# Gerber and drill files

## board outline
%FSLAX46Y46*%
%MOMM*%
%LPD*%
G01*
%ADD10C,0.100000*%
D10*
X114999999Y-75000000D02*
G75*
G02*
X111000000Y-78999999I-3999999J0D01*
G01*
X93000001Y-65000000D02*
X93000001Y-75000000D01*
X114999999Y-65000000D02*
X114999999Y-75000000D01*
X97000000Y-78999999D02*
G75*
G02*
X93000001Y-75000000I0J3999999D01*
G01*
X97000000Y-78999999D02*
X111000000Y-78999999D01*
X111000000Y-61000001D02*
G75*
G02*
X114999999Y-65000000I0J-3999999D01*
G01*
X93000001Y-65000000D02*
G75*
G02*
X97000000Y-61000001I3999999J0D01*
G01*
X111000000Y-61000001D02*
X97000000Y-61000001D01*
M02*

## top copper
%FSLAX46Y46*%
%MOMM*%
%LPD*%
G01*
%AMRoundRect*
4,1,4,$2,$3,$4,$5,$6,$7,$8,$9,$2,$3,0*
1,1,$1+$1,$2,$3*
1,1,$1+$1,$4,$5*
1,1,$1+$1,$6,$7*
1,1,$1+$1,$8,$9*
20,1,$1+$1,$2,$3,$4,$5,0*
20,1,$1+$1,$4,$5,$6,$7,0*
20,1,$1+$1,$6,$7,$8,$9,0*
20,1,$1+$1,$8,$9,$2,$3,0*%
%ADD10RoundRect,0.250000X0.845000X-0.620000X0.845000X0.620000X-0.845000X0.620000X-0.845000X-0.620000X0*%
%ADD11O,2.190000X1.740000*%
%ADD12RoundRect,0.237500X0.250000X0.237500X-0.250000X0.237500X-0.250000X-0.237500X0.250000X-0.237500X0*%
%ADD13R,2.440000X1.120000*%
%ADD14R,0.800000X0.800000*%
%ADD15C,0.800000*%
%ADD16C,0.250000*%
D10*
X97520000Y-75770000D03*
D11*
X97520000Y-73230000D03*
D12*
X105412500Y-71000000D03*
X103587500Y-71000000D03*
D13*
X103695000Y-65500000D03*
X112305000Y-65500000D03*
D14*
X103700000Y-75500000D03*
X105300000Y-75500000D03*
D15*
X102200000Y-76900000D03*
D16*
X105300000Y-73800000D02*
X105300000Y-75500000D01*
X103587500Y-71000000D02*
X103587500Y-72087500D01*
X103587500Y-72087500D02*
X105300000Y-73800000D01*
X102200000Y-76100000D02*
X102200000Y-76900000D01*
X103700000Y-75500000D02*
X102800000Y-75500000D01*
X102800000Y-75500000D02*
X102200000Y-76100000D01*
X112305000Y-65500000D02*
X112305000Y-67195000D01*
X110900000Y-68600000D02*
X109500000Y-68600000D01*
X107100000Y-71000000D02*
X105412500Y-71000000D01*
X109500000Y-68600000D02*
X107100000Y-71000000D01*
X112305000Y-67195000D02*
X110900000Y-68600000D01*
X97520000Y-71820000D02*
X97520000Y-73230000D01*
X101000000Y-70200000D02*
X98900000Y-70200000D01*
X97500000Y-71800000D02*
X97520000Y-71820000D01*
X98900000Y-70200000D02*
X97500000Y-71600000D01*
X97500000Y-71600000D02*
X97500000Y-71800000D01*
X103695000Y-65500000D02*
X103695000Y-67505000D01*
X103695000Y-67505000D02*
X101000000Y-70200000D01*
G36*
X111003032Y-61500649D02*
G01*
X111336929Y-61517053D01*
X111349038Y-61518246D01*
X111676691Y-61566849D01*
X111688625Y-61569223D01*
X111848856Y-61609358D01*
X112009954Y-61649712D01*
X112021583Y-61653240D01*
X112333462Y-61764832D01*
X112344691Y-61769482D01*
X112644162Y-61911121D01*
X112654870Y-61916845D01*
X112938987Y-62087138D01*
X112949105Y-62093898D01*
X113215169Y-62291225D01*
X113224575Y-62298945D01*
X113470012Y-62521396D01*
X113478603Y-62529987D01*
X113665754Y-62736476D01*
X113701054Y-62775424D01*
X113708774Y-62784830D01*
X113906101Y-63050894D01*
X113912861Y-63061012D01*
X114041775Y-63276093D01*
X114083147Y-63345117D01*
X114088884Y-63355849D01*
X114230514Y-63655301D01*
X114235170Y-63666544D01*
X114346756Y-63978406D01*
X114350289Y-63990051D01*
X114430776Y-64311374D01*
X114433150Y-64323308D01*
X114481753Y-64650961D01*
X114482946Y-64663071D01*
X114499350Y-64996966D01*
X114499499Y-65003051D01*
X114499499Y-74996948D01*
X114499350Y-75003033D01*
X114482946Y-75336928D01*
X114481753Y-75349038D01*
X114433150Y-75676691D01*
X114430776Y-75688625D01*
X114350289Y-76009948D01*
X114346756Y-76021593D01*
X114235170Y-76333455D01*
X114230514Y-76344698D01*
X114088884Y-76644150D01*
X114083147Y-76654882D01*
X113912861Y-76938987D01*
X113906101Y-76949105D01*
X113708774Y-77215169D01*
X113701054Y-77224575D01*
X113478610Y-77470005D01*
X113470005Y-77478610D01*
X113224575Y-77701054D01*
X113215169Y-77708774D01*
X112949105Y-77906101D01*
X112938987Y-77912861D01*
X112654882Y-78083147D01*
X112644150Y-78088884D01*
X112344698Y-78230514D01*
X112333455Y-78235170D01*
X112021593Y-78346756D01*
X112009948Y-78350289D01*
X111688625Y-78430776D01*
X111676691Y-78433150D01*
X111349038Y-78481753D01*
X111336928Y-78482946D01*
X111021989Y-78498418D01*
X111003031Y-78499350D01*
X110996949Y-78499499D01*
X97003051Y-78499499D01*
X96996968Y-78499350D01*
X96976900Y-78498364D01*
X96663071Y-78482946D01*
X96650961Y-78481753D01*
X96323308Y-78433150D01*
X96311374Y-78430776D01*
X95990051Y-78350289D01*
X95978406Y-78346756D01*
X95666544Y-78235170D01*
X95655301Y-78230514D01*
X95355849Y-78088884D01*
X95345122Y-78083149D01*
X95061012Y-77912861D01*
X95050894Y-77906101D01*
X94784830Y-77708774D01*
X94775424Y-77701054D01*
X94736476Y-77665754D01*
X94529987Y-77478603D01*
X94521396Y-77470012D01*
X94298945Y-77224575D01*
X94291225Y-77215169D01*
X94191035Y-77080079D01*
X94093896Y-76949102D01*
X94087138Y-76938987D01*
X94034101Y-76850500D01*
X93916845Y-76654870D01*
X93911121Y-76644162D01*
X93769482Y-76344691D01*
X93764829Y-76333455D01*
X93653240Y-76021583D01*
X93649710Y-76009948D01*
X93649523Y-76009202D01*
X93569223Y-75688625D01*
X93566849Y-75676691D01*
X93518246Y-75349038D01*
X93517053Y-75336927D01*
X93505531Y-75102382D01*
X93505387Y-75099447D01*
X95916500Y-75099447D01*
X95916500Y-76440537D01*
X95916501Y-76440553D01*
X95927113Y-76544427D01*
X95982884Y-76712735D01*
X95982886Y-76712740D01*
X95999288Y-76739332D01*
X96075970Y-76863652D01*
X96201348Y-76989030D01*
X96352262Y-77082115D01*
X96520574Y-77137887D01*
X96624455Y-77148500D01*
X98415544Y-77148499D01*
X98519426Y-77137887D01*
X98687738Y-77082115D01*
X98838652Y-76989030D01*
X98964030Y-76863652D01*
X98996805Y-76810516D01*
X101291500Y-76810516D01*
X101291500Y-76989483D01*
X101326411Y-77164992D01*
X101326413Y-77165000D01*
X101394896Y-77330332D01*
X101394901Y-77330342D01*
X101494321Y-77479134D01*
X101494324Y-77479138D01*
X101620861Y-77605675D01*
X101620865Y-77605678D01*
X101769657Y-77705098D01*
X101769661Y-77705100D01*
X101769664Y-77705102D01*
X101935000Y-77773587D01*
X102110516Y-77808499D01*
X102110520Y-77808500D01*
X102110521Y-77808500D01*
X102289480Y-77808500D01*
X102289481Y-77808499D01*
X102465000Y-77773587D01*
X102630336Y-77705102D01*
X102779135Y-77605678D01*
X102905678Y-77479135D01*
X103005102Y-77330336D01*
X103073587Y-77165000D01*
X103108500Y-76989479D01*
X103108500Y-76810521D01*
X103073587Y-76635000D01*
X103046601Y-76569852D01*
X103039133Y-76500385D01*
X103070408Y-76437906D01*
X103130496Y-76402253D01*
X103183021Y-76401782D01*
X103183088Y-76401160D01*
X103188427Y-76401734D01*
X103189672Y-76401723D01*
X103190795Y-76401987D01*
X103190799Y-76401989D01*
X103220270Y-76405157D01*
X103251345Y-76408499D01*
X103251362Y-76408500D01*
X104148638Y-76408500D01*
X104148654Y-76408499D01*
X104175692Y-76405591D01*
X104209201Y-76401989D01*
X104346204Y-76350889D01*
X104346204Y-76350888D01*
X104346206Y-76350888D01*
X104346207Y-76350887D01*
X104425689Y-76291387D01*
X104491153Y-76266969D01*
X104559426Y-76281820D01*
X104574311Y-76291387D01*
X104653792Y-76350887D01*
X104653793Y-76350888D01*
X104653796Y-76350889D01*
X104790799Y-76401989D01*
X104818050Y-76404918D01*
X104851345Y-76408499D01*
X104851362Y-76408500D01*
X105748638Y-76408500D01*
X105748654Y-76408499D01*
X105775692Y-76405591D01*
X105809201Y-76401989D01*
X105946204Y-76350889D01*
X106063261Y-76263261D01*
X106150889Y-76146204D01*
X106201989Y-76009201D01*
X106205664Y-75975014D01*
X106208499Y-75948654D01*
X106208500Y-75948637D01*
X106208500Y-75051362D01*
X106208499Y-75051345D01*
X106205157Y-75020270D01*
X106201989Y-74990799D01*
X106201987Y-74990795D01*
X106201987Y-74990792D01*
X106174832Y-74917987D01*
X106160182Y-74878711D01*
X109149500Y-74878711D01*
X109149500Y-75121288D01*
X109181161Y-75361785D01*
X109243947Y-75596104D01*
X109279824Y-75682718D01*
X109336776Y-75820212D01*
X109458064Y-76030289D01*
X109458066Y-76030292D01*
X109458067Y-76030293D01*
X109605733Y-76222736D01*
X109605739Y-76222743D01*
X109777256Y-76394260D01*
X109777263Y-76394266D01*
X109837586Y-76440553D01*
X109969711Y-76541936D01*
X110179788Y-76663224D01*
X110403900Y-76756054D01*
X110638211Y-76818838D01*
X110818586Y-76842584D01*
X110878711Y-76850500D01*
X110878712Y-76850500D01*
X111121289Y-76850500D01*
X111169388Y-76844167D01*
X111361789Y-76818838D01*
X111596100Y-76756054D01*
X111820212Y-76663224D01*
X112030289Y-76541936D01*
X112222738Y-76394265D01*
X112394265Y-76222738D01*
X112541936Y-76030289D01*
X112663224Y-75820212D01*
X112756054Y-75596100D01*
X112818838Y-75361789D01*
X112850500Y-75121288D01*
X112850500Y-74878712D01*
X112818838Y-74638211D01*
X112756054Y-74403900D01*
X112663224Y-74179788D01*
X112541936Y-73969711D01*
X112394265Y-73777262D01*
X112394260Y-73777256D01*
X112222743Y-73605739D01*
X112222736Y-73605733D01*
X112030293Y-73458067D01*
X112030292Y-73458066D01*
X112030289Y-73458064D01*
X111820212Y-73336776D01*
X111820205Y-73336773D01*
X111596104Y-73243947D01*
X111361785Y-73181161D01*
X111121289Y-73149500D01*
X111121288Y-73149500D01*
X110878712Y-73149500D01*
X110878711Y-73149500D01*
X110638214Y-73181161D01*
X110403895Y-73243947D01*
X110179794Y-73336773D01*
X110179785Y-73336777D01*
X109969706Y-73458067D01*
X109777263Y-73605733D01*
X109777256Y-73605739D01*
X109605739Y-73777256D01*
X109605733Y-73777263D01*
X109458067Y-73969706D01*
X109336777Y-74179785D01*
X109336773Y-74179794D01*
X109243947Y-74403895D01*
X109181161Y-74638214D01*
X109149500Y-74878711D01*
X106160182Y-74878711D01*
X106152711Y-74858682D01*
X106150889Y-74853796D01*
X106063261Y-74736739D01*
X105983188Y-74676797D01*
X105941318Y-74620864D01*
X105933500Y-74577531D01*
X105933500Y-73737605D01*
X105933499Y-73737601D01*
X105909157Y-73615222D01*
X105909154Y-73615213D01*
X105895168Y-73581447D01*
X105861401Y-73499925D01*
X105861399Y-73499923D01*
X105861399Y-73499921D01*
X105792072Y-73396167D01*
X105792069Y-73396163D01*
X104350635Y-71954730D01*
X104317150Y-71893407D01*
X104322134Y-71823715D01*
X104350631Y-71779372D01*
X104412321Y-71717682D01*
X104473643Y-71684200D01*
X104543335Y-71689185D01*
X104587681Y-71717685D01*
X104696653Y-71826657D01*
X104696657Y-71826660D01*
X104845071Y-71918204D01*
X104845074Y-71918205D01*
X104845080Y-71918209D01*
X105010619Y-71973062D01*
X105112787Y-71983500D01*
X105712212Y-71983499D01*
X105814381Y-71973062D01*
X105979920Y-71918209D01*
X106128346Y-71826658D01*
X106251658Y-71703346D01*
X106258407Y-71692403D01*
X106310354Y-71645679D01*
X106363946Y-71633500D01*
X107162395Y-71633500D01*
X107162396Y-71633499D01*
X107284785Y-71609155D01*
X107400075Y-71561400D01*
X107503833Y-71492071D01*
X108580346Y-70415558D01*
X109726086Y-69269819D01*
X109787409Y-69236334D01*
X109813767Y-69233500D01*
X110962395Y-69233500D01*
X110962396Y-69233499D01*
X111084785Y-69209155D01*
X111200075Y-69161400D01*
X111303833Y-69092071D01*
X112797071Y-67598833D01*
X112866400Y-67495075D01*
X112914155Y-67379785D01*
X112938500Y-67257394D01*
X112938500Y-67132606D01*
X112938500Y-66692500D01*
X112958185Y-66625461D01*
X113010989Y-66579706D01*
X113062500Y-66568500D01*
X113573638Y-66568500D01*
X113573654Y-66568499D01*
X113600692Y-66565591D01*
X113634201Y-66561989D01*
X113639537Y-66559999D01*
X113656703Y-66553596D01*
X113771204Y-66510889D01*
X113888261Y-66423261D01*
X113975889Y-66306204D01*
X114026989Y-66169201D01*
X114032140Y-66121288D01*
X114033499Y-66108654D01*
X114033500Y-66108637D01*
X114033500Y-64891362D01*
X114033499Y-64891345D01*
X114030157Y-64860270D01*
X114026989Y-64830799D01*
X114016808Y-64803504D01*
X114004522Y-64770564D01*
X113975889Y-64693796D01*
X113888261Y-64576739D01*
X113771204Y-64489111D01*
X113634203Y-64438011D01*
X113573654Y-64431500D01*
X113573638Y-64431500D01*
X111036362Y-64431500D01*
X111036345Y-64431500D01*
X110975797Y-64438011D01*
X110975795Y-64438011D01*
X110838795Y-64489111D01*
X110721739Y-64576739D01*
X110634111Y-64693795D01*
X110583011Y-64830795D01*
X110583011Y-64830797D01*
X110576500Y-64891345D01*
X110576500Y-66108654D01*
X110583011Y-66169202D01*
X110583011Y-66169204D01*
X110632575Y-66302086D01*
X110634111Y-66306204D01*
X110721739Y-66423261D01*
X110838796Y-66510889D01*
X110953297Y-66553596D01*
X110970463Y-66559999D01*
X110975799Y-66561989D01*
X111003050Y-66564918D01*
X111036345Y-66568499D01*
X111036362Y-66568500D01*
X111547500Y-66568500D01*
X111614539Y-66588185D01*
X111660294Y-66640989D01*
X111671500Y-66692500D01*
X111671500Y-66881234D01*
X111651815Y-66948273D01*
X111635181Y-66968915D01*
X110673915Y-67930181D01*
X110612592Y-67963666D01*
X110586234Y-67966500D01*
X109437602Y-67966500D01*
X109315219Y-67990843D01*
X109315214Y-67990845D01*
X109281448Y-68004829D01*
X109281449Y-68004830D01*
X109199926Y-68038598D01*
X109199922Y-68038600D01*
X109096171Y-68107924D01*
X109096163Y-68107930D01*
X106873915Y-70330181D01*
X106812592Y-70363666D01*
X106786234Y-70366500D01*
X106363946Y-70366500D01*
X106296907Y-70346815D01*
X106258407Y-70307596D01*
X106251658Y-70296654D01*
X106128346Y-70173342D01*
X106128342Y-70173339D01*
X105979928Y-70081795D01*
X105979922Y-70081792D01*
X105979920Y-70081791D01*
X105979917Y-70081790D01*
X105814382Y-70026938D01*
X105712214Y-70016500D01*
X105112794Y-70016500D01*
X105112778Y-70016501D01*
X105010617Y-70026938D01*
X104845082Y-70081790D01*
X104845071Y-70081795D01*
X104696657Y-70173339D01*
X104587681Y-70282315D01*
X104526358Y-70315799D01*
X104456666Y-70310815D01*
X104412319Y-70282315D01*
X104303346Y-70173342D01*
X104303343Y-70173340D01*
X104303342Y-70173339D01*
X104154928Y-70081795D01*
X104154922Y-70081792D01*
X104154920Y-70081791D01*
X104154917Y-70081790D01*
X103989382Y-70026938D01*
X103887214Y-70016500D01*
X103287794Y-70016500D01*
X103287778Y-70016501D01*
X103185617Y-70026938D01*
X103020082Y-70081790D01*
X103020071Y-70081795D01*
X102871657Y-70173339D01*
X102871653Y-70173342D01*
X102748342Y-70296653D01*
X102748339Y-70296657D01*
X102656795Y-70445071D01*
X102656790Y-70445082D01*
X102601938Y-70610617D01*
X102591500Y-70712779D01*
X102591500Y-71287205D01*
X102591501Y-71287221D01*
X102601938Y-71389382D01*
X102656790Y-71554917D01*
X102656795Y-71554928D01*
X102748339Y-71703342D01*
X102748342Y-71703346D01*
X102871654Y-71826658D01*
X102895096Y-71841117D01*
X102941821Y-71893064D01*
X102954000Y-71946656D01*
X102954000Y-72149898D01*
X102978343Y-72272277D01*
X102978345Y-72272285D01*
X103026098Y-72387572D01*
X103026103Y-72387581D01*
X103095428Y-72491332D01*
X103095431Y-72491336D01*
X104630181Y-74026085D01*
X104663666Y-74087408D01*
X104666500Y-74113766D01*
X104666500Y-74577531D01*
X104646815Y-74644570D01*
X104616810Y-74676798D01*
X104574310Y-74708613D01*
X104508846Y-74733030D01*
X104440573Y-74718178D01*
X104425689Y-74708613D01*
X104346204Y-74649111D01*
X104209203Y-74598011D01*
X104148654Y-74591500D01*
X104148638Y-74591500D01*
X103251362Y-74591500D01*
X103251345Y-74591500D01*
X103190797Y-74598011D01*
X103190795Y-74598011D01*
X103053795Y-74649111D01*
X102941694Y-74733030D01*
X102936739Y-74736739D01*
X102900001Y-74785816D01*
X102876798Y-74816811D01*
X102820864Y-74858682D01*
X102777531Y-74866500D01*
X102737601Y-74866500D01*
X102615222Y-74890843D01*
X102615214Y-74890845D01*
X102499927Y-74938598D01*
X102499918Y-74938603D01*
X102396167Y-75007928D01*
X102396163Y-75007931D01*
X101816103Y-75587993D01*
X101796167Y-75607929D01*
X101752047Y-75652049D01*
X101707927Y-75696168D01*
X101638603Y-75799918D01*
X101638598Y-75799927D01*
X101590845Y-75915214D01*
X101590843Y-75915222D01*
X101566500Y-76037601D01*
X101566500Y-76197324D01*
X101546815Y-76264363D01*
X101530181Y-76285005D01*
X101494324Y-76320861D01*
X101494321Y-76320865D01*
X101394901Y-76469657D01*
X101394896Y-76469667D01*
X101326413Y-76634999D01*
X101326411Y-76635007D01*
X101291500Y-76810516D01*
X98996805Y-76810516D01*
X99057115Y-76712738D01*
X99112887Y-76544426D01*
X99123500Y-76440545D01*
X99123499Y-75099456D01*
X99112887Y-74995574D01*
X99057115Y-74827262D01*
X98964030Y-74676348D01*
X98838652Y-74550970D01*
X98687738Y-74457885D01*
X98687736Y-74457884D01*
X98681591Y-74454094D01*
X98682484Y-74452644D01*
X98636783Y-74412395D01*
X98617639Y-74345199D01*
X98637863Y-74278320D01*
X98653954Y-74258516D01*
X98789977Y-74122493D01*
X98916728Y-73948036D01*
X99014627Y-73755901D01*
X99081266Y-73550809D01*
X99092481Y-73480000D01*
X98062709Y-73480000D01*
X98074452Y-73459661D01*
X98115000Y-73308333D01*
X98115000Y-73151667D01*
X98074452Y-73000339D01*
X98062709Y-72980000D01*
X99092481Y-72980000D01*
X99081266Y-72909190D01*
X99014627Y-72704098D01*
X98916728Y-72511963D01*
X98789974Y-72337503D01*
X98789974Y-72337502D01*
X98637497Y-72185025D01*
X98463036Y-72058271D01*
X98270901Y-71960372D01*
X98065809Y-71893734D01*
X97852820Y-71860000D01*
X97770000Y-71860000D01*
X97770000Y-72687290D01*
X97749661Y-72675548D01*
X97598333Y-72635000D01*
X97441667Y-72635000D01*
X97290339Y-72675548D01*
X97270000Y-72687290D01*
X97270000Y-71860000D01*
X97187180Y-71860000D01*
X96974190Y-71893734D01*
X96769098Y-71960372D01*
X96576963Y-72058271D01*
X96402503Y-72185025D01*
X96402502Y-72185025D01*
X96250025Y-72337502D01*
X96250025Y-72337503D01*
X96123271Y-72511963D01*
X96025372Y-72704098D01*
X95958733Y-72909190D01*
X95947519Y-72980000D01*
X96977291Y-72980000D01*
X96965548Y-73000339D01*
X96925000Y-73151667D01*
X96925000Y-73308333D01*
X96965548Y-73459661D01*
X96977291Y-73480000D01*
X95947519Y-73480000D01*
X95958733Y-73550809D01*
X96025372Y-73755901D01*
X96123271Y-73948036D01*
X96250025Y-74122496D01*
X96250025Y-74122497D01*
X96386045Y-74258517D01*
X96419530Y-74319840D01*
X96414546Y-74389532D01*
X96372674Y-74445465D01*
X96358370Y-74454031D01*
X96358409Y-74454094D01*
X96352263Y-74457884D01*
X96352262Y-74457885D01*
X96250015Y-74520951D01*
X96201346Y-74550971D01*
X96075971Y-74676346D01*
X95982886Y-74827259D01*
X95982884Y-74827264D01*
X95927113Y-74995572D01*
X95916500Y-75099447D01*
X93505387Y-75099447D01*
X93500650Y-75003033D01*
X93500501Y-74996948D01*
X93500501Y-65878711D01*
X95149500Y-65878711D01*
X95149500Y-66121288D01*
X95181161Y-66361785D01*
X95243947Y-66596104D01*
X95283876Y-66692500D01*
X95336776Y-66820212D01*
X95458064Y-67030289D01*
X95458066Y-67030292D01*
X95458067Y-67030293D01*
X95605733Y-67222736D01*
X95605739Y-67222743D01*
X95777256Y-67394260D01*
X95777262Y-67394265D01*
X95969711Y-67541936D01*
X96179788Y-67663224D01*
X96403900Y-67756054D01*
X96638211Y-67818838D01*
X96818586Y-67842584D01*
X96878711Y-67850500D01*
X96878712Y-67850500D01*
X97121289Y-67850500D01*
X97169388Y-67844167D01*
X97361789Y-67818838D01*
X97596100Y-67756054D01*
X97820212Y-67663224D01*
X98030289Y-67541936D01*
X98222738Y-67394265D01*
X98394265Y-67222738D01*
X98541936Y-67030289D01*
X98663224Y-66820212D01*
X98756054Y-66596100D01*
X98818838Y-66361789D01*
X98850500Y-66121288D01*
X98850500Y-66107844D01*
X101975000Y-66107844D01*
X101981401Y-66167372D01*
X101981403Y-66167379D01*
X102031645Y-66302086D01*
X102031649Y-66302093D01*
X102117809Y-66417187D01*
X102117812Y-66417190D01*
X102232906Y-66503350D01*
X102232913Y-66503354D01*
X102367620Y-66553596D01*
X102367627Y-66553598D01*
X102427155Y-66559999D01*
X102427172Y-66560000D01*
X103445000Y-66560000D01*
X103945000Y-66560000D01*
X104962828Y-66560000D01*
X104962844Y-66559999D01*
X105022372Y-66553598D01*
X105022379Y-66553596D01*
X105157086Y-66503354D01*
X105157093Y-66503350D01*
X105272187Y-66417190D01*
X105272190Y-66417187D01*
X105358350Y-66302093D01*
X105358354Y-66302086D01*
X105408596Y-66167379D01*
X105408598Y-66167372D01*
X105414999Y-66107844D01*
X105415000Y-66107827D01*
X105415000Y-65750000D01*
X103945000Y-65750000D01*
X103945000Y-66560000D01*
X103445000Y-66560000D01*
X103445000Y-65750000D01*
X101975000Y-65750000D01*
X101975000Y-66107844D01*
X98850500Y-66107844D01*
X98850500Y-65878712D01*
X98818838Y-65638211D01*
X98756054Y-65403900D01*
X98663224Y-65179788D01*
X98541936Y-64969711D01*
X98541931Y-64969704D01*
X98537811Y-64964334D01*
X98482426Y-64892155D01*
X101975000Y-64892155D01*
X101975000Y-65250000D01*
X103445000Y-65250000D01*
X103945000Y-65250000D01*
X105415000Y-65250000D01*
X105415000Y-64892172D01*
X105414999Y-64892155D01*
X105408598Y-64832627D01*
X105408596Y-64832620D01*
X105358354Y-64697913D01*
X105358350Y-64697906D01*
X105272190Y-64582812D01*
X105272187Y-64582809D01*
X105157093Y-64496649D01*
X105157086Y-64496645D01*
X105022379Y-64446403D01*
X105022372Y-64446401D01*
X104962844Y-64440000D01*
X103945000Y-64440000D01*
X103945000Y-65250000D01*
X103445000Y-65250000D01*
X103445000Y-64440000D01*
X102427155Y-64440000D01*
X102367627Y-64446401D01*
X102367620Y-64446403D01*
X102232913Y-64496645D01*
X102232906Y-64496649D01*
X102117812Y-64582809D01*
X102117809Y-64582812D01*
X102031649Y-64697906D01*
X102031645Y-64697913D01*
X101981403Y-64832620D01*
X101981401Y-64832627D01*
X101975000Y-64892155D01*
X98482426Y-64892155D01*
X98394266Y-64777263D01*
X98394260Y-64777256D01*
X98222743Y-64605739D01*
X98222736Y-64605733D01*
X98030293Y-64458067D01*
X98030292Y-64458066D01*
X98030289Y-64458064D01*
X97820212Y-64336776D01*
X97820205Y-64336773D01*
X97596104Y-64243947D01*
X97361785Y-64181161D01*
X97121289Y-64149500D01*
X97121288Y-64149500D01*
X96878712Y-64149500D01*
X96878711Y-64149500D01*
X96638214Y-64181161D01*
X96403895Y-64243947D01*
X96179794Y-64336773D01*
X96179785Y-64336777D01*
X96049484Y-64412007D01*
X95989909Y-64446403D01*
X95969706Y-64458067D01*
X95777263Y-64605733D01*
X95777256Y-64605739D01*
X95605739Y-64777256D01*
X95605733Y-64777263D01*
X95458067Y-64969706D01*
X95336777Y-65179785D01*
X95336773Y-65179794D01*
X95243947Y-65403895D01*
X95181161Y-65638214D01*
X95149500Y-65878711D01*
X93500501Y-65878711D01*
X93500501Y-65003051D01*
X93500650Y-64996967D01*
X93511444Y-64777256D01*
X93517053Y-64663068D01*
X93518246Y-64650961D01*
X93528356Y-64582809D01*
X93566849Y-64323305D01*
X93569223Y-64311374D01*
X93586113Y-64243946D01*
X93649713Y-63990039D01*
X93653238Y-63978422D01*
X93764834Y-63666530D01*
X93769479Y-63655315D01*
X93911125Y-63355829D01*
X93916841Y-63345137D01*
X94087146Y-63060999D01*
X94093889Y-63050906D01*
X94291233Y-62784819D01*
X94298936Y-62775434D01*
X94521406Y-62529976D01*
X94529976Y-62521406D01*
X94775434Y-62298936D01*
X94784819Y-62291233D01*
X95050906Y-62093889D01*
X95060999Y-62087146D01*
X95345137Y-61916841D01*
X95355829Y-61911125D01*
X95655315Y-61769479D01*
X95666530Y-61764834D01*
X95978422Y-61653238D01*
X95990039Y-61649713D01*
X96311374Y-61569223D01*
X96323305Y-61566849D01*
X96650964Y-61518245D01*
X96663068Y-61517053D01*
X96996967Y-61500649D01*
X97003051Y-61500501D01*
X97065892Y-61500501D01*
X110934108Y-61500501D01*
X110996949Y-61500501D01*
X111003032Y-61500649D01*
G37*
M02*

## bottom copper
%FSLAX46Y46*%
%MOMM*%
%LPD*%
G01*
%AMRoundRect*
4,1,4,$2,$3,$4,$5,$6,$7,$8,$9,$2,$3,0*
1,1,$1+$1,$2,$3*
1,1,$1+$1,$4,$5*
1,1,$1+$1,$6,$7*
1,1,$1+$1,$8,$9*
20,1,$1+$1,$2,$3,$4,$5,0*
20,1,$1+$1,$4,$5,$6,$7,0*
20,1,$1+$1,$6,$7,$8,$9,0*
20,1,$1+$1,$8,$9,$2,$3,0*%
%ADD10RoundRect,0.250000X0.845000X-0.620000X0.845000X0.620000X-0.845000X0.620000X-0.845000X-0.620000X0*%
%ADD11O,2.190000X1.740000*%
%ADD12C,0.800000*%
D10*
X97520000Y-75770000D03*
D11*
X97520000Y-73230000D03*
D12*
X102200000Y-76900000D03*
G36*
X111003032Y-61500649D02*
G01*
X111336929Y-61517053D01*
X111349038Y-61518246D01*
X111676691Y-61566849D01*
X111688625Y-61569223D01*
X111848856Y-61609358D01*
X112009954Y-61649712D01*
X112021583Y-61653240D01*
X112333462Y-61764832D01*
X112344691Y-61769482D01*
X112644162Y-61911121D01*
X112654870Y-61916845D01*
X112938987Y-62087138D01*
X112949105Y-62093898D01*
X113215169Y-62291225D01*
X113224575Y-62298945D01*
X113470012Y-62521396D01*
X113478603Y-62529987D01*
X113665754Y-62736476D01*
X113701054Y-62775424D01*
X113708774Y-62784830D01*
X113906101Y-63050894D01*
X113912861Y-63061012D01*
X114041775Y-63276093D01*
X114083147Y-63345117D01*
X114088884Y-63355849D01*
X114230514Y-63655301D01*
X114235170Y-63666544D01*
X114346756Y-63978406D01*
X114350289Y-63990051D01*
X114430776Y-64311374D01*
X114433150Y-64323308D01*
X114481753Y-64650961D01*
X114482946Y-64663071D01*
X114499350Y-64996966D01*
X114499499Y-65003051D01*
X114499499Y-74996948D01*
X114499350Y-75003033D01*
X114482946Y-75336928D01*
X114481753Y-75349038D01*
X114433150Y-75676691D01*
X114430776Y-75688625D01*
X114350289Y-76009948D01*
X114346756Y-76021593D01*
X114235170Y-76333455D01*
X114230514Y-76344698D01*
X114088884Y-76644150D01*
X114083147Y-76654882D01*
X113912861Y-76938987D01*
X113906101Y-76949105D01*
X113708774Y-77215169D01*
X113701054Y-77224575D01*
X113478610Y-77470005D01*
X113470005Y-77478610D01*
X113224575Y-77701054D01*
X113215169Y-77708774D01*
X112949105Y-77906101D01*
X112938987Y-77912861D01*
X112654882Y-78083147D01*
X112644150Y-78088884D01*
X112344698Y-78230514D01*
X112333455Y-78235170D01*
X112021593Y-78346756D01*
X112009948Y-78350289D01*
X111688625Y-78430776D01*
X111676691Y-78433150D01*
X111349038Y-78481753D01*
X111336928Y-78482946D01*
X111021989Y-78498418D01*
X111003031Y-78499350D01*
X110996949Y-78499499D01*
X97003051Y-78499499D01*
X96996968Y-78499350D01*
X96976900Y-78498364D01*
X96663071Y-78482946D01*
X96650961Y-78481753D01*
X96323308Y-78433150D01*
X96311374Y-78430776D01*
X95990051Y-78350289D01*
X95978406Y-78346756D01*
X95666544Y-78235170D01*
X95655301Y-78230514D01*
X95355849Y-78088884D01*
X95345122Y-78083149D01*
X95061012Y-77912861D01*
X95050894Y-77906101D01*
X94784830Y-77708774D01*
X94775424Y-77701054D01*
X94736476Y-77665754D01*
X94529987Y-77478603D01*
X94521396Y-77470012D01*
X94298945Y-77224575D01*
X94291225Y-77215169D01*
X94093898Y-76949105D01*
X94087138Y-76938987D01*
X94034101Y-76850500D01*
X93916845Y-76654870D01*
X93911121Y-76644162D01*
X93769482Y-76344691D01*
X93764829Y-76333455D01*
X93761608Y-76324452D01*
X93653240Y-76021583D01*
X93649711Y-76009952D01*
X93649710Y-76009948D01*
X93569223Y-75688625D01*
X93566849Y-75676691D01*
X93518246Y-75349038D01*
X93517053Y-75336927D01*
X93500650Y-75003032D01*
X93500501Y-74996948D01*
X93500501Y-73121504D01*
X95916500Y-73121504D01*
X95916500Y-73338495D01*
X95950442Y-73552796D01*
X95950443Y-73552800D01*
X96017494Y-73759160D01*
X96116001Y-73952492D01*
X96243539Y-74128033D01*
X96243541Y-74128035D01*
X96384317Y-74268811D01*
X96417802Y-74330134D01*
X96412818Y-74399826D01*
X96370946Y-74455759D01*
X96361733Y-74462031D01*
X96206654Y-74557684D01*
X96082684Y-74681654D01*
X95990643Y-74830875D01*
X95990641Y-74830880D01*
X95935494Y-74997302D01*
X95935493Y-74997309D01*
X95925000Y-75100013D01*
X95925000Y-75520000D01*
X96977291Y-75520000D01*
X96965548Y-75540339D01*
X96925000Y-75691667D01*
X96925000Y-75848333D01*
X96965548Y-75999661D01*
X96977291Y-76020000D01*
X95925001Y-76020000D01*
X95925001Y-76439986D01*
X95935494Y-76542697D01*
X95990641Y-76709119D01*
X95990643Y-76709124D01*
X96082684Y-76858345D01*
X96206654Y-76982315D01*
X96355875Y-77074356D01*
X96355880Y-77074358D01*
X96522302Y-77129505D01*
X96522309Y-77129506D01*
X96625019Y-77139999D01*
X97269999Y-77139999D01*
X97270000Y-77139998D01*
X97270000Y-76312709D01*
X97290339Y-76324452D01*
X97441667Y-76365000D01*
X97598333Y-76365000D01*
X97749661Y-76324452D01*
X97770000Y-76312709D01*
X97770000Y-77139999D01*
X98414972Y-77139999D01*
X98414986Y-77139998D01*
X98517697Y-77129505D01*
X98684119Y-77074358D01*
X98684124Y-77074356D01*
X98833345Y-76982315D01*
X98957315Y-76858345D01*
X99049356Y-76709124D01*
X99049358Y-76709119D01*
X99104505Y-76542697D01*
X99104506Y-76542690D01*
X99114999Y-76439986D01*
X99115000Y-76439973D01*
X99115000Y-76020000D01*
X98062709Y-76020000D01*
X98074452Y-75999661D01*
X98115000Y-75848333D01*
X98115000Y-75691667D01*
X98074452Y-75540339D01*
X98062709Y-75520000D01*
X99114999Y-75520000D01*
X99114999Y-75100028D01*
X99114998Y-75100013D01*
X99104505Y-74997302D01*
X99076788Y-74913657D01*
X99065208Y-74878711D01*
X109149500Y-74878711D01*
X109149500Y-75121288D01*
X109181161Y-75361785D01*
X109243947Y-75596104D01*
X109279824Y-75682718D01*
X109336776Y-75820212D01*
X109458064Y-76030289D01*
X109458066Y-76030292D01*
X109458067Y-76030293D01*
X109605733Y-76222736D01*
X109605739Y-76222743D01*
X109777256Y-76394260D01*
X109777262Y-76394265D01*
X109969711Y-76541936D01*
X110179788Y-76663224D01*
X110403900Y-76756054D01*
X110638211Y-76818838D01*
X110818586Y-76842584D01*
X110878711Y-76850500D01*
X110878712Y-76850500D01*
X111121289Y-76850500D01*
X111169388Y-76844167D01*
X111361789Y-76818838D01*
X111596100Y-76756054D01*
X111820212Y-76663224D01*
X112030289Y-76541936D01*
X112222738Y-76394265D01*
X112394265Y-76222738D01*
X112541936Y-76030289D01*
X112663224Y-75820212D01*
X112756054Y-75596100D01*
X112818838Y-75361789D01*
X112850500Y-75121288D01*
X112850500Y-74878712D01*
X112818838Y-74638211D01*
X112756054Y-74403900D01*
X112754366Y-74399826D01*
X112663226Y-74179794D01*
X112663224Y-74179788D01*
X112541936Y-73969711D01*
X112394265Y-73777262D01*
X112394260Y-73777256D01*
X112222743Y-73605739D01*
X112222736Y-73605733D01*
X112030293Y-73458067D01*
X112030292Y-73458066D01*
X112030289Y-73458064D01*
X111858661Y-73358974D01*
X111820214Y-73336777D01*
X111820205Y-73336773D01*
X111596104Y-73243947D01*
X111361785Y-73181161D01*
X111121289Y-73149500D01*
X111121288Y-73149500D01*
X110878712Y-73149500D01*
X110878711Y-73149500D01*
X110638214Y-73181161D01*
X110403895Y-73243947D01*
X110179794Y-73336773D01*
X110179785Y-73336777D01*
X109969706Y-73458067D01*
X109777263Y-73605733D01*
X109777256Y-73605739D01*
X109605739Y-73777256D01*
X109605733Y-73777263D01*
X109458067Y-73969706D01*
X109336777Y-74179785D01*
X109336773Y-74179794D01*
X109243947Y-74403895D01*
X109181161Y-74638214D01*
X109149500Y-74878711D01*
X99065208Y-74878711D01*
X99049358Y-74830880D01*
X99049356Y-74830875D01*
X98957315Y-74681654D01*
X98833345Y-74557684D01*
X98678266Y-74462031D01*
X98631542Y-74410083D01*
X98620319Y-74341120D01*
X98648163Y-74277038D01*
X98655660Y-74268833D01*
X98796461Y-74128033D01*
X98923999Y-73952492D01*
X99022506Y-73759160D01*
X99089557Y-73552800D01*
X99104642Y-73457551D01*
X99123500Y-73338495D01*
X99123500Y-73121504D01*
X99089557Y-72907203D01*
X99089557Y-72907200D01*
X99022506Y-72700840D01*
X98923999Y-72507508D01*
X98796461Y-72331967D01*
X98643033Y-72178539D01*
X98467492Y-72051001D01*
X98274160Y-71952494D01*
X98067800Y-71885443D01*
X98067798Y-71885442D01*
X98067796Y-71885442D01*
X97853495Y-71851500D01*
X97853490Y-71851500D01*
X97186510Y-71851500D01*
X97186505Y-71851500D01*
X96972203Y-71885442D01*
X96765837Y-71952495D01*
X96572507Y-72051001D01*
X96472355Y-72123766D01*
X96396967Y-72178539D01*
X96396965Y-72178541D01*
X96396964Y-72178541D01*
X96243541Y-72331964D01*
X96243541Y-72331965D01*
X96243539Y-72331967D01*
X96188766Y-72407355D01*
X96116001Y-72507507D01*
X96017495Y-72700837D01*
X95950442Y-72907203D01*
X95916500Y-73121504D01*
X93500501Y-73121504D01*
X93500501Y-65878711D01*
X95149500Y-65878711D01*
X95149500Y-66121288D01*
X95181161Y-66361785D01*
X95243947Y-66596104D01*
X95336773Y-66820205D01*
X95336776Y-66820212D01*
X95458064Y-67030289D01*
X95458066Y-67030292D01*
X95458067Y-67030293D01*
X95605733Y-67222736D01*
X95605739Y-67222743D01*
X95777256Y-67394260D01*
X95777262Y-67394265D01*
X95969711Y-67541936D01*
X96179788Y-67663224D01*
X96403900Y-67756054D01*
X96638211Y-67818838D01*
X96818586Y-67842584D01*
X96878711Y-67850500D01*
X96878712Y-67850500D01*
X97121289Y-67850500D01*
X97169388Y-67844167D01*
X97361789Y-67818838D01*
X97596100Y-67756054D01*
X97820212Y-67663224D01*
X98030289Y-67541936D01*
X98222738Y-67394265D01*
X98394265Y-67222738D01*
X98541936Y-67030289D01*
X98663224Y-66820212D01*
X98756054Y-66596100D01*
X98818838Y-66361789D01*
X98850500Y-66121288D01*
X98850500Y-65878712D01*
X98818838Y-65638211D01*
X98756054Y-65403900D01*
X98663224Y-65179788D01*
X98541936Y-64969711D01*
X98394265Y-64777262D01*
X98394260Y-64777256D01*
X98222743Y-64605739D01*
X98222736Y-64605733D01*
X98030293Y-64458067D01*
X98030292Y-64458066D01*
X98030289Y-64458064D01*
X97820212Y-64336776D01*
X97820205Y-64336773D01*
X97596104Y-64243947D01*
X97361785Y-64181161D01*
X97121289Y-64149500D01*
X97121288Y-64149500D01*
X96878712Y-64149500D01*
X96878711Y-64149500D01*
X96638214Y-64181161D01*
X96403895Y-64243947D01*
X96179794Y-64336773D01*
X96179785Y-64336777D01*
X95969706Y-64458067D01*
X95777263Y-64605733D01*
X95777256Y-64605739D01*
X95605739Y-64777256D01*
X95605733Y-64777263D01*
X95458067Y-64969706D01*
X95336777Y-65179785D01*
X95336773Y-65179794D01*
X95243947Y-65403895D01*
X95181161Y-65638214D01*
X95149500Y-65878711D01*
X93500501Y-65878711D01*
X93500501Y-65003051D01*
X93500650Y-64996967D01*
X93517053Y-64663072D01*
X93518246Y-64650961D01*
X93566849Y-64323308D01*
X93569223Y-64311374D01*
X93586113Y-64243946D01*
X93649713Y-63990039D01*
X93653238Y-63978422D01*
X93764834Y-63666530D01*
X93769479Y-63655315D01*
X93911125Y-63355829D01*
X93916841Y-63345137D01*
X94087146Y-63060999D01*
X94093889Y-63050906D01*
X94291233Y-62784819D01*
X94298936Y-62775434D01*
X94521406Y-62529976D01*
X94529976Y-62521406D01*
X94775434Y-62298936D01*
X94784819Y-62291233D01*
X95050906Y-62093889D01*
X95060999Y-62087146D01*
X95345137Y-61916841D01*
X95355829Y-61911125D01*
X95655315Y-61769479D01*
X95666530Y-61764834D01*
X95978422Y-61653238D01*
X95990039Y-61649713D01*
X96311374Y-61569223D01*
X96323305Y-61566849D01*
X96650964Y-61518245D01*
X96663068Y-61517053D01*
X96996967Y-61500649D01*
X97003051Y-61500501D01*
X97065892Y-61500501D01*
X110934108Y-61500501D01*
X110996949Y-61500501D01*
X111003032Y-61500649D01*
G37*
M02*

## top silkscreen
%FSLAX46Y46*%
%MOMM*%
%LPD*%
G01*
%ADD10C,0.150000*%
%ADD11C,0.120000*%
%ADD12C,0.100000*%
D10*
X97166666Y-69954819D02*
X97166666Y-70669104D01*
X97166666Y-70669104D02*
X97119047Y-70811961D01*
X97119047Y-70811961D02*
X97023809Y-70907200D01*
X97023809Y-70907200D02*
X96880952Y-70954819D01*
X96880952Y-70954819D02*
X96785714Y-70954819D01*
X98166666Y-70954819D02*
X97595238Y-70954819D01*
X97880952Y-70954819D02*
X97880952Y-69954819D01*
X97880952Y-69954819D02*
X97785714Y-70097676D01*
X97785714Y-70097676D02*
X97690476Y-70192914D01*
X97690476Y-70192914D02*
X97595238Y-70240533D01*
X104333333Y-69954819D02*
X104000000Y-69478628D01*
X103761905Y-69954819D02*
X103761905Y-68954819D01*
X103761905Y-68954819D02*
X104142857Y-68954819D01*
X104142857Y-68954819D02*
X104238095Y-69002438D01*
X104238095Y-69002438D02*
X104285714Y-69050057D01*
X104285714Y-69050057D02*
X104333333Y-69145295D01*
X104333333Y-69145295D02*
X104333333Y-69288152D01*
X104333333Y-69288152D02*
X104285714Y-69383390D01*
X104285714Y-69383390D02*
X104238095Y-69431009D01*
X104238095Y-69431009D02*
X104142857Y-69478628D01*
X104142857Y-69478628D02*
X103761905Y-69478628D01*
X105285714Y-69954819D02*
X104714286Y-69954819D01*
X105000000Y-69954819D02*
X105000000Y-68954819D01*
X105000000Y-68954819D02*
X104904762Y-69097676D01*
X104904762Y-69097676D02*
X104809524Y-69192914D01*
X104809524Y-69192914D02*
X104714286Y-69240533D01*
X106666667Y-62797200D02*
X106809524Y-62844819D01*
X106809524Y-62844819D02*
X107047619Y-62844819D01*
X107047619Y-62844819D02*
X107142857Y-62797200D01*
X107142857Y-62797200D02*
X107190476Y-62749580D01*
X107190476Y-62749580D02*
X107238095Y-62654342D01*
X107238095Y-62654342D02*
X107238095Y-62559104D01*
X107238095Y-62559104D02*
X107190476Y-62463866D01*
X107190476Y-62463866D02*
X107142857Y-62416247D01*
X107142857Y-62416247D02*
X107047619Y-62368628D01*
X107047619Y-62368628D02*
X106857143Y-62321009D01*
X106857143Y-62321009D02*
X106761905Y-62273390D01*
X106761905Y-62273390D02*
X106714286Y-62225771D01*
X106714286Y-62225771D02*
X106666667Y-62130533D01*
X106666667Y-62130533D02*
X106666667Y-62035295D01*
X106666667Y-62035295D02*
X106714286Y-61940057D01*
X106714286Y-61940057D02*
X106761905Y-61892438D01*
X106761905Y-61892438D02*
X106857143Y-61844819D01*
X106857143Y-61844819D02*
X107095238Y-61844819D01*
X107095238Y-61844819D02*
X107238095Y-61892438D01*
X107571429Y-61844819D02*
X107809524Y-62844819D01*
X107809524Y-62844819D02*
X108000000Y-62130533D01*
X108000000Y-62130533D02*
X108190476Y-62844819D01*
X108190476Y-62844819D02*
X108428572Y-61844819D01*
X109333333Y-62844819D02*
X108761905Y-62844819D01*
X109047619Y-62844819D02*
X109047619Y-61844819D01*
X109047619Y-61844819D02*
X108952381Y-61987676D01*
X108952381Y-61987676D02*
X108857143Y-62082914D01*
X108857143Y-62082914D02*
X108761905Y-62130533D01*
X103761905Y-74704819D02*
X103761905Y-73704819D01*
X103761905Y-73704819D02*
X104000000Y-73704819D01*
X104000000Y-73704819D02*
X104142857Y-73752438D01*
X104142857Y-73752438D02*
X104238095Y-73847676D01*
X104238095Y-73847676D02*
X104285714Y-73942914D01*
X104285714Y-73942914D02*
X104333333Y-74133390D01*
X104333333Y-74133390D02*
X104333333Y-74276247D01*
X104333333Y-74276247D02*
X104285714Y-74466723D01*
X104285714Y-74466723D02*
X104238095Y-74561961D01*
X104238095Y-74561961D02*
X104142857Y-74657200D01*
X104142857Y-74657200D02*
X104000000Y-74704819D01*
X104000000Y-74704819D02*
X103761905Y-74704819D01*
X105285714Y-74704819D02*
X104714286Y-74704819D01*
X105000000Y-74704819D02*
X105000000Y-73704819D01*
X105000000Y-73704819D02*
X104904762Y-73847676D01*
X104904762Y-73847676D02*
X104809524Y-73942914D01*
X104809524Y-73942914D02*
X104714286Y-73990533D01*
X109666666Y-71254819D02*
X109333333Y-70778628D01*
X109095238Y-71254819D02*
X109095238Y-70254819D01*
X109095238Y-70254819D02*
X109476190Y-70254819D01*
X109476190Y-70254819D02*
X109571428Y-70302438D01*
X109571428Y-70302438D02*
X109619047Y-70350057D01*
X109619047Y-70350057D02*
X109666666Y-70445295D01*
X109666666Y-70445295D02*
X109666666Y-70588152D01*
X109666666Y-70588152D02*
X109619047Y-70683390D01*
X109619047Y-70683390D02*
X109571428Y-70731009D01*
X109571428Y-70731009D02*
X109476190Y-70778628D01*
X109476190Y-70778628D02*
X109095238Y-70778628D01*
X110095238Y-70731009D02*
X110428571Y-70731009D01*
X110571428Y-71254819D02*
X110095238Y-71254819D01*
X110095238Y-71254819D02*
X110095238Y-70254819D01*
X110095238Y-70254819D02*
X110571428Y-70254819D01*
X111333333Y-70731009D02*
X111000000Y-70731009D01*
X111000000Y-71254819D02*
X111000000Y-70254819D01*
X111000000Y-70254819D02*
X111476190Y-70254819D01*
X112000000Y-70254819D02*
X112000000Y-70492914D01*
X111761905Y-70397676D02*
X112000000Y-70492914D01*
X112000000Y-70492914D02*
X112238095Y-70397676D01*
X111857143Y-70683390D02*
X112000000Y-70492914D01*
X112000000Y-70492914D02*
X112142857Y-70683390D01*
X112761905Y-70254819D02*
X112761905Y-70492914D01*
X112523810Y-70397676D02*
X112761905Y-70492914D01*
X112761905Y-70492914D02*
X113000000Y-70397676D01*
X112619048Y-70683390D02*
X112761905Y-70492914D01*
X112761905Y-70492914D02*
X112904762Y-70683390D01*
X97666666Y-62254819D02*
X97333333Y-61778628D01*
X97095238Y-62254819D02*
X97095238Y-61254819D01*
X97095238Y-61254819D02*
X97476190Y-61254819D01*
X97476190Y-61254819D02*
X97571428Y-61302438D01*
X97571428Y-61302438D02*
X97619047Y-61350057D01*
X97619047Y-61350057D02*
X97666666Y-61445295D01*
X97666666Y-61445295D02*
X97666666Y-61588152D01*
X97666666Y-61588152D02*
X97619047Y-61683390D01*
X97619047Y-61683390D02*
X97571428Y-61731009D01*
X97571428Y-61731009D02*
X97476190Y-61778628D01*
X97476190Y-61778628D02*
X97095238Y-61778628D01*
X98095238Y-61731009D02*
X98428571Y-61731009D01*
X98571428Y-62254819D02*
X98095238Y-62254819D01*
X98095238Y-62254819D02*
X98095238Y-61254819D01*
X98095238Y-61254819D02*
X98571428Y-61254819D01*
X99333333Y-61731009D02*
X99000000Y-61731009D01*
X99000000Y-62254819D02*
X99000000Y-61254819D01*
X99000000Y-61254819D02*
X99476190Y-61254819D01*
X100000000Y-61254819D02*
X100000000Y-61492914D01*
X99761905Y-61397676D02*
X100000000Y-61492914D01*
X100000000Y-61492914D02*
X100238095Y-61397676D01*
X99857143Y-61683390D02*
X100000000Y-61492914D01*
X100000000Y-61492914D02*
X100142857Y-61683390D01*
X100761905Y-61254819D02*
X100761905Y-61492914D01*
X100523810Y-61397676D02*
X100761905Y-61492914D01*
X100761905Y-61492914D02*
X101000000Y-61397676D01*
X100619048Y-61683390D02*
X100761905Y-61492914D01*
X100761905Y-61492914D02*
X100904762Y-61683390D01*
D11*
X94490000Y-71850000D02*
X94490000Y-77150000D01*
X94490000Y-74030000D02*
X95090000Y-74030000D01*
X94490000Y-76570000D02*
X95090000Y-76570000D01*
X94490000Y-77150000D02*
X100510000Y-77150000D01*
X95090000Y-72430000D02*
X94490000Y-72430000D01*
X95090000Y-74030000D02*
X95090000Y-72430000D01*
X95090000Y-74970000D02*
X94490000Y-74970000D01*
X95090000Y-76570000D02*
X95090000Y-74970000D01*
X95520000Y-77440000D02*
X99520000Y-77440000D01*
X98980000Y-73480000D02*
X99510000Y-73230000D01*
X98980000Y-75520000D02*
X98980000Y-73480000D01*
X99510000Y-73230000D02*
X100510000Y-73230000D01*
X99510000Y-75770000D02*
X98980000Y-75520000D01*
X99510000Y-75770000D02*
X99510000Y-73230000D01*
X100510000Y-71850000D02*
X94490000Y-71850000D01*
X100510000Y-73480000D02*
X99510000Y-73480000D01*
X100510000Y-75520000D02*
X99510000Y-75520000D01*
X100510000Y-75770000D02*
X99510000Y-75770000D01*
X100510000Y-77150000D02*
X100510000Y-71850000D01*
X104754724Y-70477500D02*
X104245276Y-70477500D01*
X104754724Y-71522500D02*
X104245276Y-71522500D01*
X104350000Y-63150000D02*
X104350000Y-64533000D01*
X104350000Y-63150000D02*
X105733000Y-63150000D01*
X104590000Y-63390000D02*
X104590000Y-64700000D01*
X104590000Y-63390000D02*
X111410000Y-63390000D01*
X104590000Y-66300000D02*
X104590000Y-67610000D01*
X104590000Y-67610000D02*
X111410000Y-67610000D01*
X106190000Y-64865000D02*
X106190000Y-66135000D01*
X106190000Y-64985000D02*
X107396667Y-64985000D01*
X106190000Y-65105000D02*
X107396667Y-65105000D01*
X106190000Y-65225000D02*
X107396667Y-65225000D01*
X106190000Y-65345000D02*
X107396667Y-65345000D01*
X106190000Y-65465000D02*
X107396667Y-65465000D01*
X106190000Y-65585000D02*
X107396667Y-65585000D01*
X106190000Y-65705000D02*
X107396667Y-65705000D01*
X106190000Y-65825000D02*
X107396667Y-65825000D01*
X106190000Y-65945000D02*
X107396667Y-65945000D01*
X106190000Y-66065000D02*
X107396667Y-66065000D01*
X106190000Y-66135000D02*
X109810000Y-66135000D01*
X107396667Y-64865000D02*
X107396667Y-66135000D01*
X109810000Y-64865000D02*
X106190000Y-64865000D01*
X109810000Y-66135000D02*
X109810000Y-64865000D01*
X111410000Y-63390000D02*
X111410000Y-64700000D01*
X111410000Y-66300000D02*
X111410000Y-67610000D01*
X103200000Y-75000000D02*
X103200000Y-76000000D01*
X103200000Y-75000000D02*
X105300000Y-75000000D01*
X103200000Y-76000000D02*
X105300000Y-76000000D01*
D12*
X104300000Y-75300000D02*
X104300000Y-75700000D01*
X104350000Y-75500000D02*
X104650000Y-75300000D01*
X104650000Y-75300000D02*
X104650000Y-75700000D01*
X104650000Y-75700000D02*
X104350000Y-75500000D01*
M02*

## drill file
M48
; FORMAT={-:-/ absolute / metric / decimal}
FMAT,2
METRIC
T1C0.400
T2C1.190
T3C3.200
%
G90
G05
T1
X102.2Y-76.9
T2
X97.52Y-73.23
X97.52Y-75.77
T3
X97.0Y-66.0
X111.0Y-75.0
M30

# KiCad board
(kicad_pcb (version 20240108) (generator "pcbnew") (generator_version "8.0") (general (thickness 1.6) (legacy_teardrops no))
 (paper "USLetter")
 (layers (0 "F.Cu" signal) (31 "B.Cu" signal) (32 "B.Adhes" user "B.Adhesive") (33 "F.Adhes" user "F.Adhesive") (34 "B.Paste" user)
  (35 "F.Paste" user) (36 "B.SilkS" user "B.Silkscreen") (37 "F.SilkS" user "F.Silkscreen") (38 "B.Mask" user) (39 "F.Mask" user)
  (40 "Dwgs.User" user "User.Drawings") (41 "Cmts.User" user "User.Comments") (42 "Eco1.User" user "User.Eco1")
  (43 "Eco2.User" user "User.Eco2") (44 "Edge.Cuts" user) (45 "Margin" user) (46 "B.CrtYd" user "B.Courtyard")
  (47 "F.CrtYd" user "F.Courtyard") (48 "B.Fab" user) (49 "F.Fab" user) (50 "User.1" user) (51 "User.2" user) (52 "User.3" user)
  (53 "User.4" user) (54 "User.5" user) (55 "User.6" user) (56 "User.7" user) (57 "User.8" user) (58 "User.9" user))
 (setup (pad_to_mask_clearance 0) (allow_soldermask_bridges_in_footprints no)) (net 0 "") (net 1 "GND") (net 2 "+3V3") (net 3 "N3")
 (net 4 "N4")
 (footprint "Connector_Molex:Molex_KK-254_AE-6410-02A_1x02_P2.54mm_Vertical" (layer "F.Cu") (at 97.52 75.77 90)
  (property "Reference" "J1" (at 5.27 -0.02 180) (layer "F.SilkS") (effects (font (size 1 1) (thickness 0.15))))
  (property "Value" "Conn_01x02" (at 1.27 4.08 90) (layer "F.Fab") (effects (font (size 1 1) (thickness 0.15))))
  (fp_line (start 3.92 -3.03) (end -1.38 -3.03) (stroke (width 0.12) (type solid)) (layer "F.SilkS"))
  (fp_line (start 1.74 -3.03) (end 1.74 -2.43) (stroke (width 0.12) (type solid)) (layer "F.SilkS"))
  (fp_line (start -0.8 -3.03) (end -0.8 -2.43) (stroke (width 0.12) (type solid)) (layer "F.SilkS"))
  (fp_line (start -1.38 -3.03) (end -1.38 2.99) (stroke (width 0.12) (type solid)) (layer "F.SilkS"))
  (fp_line (start 3.34 -2.43) (end 3.34 -3.03) (stroke (width 0.12) (type solid)) (layer "F.SilkS"))
  (fp_line (start 1.74 -2.43) (end 3.34 -2.43) (stroke (width 0.12) (type solid)) (layer "F.SilkS"))
  (fp_line (start 0.8 -2.43) (end 0.8 -3.03) (stroke (width 0.12) (type solid)) (layer "F.SilkS"))
  (fp_line (start -0.8 -2.43) (end 0.8 -2.43) (stroke (width 0.12) (type solid)) (layer "F.SilkS"))
  (fp_line (start -1.67 -2) (end -1.67 2) (stroke (width 0.12) (type solid)) (layer "F.SilkS"))
  (fp_line (start 2.29 1.46) (end 2.54 1.99) (stroke (width 0.12) (type solid)) (layer "F.SilkS"))
  (fp_line (start 0.25 1.46) (end 2.29 1.46) (stroke (width 0.12) (type solid)) (layer "F.SilkS"))
  (fp_line (start 2.54 1.99) (end 2.54 2.99) (stroke (width 0.12) (type solid)) (layer "F.SilkS"))
  (fp_line (start 0 1.99) (end 0.25 1.46) (stroke (width 0.12) (type solid)) (layer "F.SilkS"))
  (fp_line (start 0 1.99) (end 2.54 1.99) (stroke (width 0.12) (type solid)) (layer "F.SilkS"))
  (fp_line (start 3.92 2.99) (end 3.92 -3.03) (stroke (width 0.12) (type solid)) (layer "F.SilkS"))
  (fp_line (start 2.29 2.99) (end 2.29 1.99) (stroke (width 0.12) (type solid)) (layer "F.SilkS"))
  (fp_line (start 0.25 2.99) (end 0.25 1.99) (stroke (width 0.12) (type solid)) (layer "F.SilkS"))
  (fp_line (start 0 2.99) (end 0 1.99) (stroke (width 0.12) (type solid)) (layer "F.SilkS"))
  (fp_line (start -1.38 2.99) (end 3.92 2.99) (stroke (width 0.12) (type solid)) (layer "F.SilkS"))
  (pad "1" thru_hole roundrect (at 0 0 90) (size 1.74 2.19) (drill 1.19) (layers "*.Cu" "*.Mask") (remove_unused_layers no)
   (roundrect_rratio 0.143678) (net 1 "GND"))
  (pad "2" thru_hole oval (at 2.54 0 90) (size 1.74 2.19) (drill 1.19) (layers "*.Cu" "*.Mask") (remove_unused_layers no) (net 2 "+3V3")))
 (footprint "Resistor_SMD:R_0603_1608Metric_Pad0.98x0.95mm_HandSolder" (layer "F.Cu") (at 104.5 71 180)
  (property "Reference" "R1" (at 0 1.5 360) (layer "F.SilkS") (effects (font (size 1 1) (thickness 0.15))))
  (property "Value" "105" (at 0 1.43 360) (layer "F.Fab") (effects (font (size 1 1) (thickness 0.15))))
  (fp_line (start -0.254724 0.5225) (end 0.254724 0.5225) (stroke (width 0.12) (type solid)) (layer "F.SilkS"))
  (fp_line (start -0.254724 -0.5225) (end 0.254724 -0.5225) (stroke (width 0.12) (type solid)) (layer "F.SilkS"))
  (pad "1" smd roundrect (at -0.9125 0 180) (size 0.975 0.95) (layers "F.Cu" "F.Paste" "F.Mask") (roundrect_rratio 0.25) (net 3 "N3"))
  (pad "2" smd roundrect (at 0.9125 0 180) (size 0.975 0.95) (layers "F.Cu" "F.Paste" "F.Mask") (roundrect_rratio 0.25) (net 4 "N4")))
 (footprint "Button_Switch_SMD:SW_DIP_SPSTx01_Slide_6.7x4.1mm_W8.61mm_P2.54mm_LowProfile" (layer "F.Cu") (at 108 65.5)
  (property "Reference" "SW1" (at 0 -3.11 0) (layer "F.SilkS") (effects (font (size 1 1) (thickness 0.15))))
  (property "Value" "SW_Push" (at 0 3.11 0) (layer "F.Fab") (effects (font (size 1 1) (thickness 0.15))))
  (fp_line (start -3.65 -2.35) (end -3.65 -0.967) (stroke (width 0.12) (type solid)) (layer "F.SilkS"))
  (fp_line (start -3.65 -2.35) (end -2.267 -2.35) (stroke (width 0.12) (type solid)) (layer "F.SilkS"))
  (fp_line (start -3.41 -2.11) (end -3.41 -0.8) (stroke (width 0.12) (type solid)) (layer "F.SilkS"))
  (fp_line (start -3.41 -2.11) (end 3.41 -2.11) (stroke (width 0.12) (type solid)) (layer "F.SilkS"))
  (fp_line (start -3.41 0.8) (end -3.41 2.11) (stroke (width 0.12) (type solid)) (layer "F.SilkS"))
  (fp_line (start -3.41 2.11) (end 3.41 2.11) (stroke (width 0.12) (type solid)) (layer "F.SilkS"))
  (fp_line (start -1.81 -0.635) (end -1.81 0.635) (stroke (width 0.12) (type solid)) (layer "F.SilkS"))
  (fp_line (start -1.81 -0.515) (end -0.603333 -0.515) (stroke (width 0.12) (type solid)) (layer "F.SilkS"))
  (fp_line (start -1.81 -0.395) (end -0.603333 -0.395) (stroke (width 0.12) (type solid)) (layer "F.SilkS"))
  (fp_line (start -1.81 -0.275) (end -0.603333 -0.275) (stroke (width 0.12) (type solid)) (layer "F.SilkS"))
  (fp_line (start -1.81 -0.155) (end -0.603333 -0.155) (stroke (width 0.12) (type solid)) (layer "F.SilkS"))
  (fp_line (start -1.81 -0.035) (end -0.603333 -0.035) (stroke (width 0.12) (type solid)) (layer "F.SilkS"))
  (fp_line (start -1.81 0.085) (end -0.603333 0.085) (stroke (width 0.12) (type solid)) (layer "F.SilkS"))
  (fp_line (start -1.81 0.205) (end -0.603333 0.205) (stroke (width 0.12) (type solid)) (layer "F.SilkS"))
  (fp_line (start -1.81 0.325) (end -0.603333 0.325) (stroke (width 0.12) (type solid)) (layer "F.SilkS"))
  (fp_line (start -1.81 0.445) (end -0.603333 0.445) (stroke (width 0.12) (type solid)) (layer "F.SilkS"))
  (fp_line (start -1.81 0.565) (end -0.603333 0.565) (stroke (width 0.12) (type solid)) (layer "F.SilkS"))
  (fp_line (start -1.81 0.635) (end 1.81 0.635) (stroke (width 0.12) (type solid)) (layer "F.SilkS"))
  (fp_line (start -0.603333 -0.635) (end -0.603333 0.635) (stroke (width 0.12) (type solid)) (layer "F.SilkS"))
  (fp_line (start 1.81 -0.635) (end -1.81 -0.635) (stroke (width 0.12) (type solid)) (layer "F.SilkS"))
  (fp_line (start 1.81 0.635) (end 1.81 -0.635) (stroke (width 0.12) (type solid)) (layer "F.SilkS"))
  (fp_line (start 3.41 -2.11) (end 3.41 -0.8) (stroke (width 0.12) (type solid)) (layer "F.SilkS"))
  (fp_line (start 3.41 0.8) (end 3.41 2.11) (stroke (width 0.12) (type solid)) (layer "F.SilkS"))
  (pad "1" smd rect (at -4.305 0) (size 2.44 1.12) (layers "F.Cu" "F.Paste" "F.Mask") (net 2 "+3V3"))
  (pad "2" smd rect (at 4.305 0) (size 2.44 1.12) (layers "F.Cu" "F.Paste" "F.Mask") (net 3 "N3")))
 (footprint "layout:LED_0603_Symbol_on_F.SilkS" (layer "F.Cu") (at 104.5 75.5)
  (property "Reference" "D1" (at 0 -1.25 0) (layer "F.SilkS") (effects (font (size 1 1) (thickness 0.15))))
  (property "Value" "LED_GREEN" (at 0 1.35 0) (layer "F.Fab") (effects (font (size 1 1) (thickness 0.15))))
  (fp_line (start -1.3 -0.5) (end -1.3 0.5) (stroke (width 0.12) (type solid)) (layer "F.SilkS"))
  (fp_line (start -1.3 -0.5) (end 0.8 -0.5) (stroke (width 0.12) (type solid)) (layer "F.SilkS"))
  (fp_line (start -1.3 0.5) (end 0.8 0.5) (stroke (width 0.12) (type solid)) (layer "F.SilkS"))
  (fp_line (start -0.2 -0.2) (end -0.2 0.2) (stroke (width 0.1) (type solid)) (layer "F.SilkS"))
  (fp_line (start -0.15 0) (end 0.15 -0.2) (stroke (width 0.1) (type solid)) (layer "F.SilkS"))
  (fp_line (start 0.15 -0.2) (end 0.15 0.2) (stroke (width 0.1) (type solid)) (layer "F.SilkS"))
  (fp_line (start 0.15 0.2) (end -0.15 0) (stroke (width 0.1) (type solid)) (layer "F.SilkS"))
  (pad "1" smd rect (at -0.8 0 180) (size 0.8 0.8) (layers "F.Cu" "F.Paste" "F.Mask") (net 1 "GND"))
  (pad "2" smd rect (at 0.8 0 180) (size 0.8 0.8) (layers "F.Cu" "F.Paste" "F.Mask") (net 4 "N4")))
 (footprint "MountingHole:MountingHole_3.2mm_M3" (layer "F.Cu") (at 111 75)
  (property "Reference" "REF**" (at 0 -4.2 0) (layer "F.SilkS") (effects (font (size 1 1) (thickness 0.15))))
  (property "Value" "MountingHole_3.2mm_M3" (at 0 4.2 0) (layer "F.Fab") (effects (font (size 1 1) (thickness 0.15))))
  (pad "" np_thru_hole circle (at 0 0) (size 3.2 3.2) (drill 3.2) (layers "*.Cu" "*.Mask")))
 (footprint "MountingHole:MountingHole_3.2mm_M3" (layer "F.Cu") (at 97 66)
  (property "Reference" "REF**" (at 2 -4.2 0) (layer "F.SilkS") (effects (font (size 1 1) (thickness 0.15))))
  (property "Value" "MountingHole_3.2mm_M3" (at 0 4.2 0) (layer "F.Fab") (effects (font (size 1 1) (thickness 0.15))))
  (pad "" np_thru_hole circle (at 0 0) (size 3.2 3.2) (drill 3.2) (layers "*.Cu" "*.Mask")))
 (gr_arc (start 114.999999 75) (mid 113.828426 77.828426) (end 111 78.999999) (stroke (width 0.1) (type default)) (layer "Edge.Cuts"))
 (gr_line (start 93.000001 65) (end 93.000001 75) (stroke (width 0.1) (type default)) (layer "Edge.Cuts"))
 (gr_line (start 114.999999 65) (end 114.999999 75) (stroke (width 0.1) (type default)) (layer "Edge.Cuts"))
 (gr_arc (start 97 78.999999) (mid 94.171574 77.828426) (end 93.000001 75) (stroke (width 0.1) (type default)) (layer "Edge.Cuts"))
 (gr_line (start 97 78.999999) (end 111 78.999999) (stroke (width 0.1) (type default)) (layer "Edge.Cuts"))
 (gr_arc (start 111 61.000001) (mid 113.828426 62.171574) (end 114.999999 65) (stroke (width 0.1) (type default)) (layer "Edge.Cuts"))
 (gr_arc (start 93.000001 65) (mid 94.171574 62.171574) (end 97 61.000001) (stroke (width 0.1) (type default)) (layer "Edge.Cuts"))
 (gr_line (start 111 61.000001) (end 97 61.000001) (stroke (width 0.1) (type default)) (layer "Edge.Cuts"))
 (segment (start 105.3 73.8) (end 105.3 75.5) (width 0.25) (layer "F.Cu") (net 4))
 (segment (start 103.5875 71) (end 103.5875 72.0875) (width 0.25) (layer "F.Cu") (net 4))
 (segment (start 103.5875 72.0875) (end 105.3 73.8) (width 0.25) (layer "F.Cu") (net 4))
 (segment (start 102.2 76.1) (end 102.2 76.9) (width 0.25) (layer "F.Cu") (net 1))
 (segment (start 103.7 75.5) (end 102.8 75.5) (width 0.25) (layer "F.Cu") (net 1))
 (segment (start 102.8 75.5) (end 102.2 76.1) (width 0.25) (layer "F.Cu") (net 1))
 (via (at 102.2 76.9) (size 0.8) (drill 0.4) (layers "F.Cu" "B.Cu") (free yes) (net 1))
 (segment (start 112.305 65.5) (end 112.305 67.195) (width 0.25) (layer "F.Cu") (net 3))
 (segment (start 110.9 68.6) (end 109.5 68.6) (width 0.25) (layer "F.Cu") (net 3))
 (segment (start 107.1 71) (end 105.4125 71) (width 0.25) (layer "F.Cu") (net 3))
 (segment (start 109.5 68.6) (end 107.1 71) (width 0.25) (layer "F.Cu") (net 3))
 (segment (start 112.305 67.195) (end 110.9 68.6) (width 0.25) (layer "F.Cu") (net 3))
 (segment (start 97.52 71.82) (end 97.52 73.23) (width 0.25) (layer "F.Cu") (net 2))
 (segment (start 101 70.2) (end 98.9 70.2) (width 0.25) (layer "F.Cu") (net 2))
 (segment (start 97.5 71.8) (end 97.52 71.82) (width 0.25) (layer "F.Cu") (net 2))
 (segment (start 98.9 70.2) (end 97.5 71.6) (width 0.25) (layer "F.Cu") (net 2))
 (segment (start 97.5 71.6) (end 97.5 71.8) (width 0.25) (layer "F.Cu") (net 2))
 (segment (start 103.695 65.5) (end 103.695 67.505) (width 0.25) (layer "F.Cu") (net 2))
 (segment (start 103.695 67.505) (end 101 70.2) (width 0.25) (layer "F.Cu") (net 2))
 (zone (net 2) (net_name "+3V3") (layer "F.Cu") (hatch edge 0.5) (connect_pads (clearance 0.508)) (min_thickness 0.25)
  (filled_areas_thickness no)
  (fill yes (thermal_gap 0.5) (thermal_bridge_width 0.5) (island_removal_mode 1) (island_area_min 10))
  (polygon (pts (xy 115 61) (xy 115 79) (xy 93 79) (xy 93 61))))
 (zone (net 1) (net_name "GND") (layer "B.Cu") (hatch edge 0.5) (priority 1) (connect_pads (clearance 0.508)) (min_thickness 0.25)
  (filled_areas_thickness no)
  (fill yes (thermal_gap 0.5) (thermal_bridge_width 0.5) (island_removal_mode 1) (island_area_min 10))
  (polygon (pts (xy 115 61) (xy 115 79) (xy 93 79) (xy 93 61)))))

